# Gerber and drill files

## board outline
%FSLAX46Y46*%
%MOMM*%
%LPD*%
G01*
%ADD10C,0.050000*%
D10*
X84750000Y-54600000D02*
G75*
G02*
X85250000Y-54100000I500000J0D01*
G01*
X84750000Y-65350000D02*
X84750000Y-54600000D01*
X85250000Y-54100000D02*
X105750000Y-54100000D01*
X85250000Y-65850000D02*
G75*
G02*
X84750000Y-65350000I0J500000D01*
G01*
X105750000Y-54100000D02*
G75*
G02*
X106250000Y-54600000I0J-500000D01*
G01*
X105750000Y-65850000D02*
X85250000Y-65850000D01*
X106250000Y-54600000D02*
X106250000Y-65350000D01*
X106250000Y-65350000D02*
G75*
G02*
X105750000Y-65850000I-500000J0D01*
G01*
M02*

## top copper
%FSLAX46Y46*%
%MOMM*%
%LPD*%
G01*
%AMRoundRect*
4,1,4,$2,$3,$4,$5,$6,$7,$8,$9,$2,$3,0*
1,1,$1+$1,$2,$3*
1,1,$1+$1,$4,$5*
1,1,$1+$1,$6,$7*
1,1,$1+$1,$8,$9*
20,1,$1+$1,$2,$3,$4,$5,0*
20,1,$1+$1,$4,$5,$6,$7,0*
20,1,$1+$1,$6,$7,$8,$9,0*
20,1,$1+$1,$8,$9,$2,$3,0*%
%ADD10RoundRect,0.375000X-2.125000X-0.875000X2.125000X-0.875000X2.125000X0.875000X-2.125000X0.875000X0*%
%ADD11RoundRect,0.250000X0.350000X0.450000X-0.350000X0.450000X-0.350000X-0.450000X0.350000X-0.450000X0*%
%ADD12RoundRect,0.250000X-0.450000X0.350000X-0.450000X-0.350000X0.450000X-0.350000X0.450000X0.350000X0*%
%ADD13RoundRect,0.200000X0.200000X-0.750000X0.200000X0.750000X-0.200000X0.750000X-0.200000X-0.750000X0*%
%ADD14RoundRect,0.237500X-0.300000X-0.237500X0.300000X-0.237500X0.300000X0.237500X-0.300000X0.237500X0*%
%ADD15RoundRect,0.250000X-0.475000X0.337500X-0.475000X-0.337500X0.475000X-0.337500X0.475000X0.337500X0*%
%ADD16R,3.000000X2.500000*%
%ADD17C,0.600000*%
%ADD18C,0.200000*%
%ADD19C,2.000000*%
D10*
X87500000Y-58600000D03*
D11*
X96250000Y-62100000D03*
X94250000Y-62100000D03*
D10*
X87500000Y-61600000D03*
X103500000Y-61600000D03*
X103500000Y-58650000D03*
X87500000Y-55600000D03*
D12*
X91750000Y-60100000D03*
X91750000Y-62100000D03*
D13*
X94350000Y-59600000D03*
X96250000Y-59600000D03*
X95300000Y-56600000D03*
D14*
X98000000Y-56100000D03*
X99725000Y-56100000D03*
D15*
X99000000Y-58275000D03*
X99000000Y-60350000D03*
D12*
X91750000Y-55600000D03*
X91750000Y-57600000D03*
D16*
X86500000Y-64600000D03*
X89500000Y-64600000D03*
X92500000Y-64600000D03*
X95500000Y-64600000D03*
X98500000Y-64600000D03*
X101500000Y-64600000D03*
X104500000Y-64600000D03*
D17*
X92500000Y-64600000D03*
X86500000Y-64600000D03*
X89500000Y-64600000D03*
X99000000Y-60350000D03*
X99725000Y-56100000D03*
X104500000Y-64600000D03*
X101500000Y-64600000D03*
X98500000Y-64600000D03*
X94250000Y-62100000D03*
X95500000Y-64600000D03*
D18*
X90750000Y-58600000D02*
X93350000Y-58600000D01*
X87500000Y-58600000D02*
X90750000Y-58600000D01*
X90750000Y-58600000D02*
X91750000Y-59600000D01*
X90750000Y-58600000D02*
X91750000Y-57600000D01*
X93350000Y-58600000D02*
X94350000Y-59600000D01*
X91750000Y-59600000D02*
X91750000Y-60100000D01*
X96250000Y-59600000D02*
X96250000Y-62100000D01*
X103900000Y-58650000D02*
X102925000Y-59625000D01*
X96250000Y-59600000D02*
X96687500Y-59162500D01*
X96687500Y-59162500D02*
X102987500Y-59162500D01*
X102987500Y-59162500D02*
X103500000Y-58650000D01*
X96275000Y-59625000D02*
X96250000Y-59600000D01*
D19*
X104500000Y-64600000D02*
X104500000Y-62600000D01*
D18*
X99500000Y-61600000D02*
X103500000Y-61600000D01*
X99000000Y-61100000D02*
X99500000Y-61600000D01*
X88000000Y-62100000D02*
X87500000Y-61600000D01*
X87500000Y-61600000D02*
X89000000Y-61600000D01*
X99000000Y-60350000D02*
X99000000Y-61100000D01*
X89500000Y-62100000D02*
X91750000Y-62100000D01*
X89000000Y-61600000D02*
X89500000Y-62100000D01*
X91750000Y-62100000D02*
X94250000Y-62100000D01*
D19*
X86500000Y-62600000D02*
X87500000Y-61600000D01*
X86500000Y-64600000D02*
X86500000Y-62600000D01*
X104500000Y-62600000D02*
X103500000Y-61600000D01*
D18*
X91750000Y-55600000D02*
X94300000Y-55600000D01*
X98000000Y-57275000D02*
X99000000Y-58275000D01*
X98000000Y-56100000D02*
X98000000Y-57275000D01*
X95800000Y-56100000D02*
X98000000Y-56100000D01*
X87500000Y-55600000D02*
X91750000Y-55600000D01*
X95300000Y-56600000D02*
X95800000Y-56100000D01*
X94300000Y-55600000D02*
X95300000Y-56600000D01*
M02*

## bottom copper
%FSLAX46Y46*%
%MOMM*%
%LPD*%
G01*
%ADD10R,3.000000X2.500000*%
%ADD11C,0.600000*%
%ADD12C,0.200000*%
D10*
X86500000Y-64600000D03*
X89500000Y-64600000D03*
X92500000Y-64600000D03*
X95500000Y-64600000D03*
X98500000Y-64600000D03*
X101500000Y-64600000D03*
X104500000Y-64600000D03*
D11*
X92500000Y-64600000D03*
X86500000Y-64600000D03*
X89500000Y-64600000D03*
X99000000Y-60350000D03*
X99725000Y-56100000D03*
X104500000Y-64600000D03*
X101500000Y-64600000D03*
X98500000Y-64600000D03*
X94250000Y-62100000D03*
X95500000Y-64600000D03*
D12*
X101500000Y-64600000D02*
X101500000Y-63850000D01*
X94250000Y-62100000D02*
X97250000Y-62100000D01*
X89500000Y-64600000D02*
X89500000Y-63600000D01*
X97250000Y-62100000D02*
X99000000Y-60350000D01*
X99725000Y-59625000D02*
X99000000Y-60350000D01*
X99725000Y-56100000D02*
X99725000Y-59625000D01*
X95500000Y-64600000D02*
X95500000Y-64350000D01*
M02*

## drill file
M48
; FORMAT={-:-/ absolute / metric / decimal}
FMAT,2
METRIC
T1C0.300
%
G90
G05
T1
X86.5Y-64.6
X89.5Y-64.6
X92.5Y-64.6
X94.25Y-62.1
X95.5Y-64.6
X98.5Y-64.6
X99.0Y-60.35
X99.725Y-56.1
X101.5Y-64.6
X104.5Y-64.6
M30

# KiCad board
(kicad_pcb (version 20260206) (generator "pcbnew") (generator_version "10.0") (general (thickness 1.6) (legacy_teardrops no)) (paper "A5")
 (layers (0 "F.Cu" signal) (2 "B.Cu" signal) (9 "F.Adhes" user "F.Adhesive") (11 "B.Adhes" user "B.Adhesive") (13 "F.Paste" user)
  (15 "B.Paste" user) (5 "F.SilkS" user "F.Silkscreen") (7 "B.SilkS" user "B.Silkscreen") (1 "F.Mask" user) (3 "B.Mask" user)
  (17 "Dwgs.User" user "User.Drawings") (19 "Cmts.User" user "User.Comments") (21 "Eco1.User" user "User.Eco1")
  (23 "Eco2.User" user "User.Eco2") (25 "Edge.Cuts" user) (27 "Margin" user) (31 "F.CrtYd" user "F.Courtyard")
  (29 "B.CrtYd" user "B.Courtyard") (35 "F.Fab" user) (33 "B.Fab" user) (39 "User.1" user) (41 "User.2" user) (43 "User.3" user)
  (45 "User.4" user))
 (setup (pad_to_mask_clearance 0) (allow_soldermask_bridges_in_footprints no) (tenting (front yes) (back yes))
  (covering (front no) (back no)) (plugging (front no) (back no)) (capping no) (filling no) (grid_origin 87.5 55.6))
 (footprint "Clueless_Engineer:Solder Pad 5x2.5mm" (layer "F.Cu") (at 87.5 58.6)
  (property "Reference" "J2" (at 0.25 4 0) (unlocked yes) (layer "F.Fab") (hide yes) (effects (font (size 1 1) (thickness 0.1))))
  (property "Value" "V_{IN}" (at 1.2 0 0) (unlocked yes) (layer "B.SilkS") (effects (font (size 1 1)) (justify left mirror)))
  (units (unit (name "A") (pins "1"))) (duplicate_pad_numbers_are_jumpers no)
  (pad "1" smd roundrect (at 0 0) (size 5 2.5) (layers "F.Cu" "F.Mask" "F.Paste") (roundrect_rratio 0.15) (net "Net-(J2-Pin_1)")))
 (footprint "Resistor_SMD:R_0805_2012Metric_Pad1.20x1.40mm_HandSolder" (layer "F.Cu") (at 95.25 62.1 180)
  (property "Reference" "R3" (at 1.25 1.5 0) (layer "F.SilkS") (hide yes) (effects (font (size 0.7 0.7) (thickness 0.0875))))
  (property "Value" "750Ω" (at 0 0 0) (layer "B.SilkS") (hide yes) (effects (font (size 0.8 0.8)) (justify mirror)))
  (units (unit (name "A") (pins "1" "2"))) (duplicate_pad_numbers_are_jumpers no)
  (pad "1" smd roundrect (at -1 0 180) (size 1.2 1.4) (layers "F.Cu" "F.Mask" "F.Paste") (roundrect_rratio 0.208333) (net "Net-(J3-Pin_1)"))
  (pad "2" smd roundrect (at 1 0 180) (size 1.2 1.4) (layers "F.Cu" "F.Mask" "F.Paste") (roundrect_rratio 0.208333) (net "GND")))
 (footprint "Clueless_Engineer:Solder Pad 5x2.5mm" (layer "F.Cu") (at 87.5 61.6)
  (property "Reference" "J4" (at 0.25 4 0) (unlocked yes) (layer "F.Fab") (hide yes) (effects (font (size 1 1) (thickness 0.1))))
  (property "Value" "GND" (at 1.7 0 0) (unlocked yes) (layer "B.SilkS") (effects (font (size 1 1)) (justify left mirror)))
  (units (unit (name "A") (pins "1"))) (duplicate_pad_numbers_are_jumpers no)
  (pad "1" smd roundrect (at 0 0) (size 5 2.5) (layers "F.Cu" "F.Mask" "F.Paste") (roundrect_rratio 0.15) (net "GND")))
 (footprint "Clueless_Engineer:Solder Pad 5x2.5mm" (layer "F.Cu") (at 103.5 61.6)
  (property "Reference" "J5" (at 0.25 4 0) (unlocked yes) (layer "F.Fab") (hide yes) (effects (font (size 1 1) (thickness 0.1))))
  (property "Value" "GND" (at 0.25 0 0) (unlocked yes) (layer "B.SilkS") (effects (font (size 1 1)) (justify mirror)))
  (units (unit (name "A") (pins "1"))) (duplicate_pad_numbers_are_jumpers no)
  (pad "1" smd roundrect (at 0 0) (size 5 2.5) (layers "F.Cu" "F.Mask" "F.Paste") (roundrect_rratio 0.15) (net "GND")))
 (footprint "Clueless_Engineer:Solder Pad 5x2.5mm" (layer "F.Cu") (at 103.6 58.85)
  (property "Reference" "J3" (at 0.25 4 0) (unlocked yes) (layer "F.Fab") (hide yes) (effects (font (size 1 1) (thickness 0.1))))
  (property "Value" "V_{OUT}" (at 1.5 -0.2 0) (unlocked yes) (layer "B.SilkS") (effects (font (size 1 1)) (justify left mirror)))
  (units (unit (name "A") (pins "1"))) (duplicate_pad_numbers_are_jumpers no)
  (pad "1" smd roundrect (at -0.1 -0.2) (size 5 2.5) (layers "F.Cu" "F.Mask" "F.Paste") (roundrect_rratio 0.15) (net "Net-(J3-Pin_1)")))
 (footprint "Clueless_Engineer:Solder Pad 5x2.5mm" (layer "F.Cu") (at 87.5 55.6)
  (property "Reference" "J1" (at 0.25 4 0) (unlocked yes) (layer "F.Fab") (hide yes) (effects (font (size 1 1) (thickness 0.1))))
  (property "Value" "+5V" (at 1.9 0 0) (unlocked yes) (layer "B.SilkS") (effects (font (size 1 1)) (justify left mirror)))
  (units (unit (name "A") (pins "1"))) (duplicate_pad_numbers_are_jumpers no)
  (pad "1" smd roundrect (at 0 0) (size 5 2.5) (layers "F.Cu" "F.Mask" "F.Paste") (roundrect_rratio 0.15) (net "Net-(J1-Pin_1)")))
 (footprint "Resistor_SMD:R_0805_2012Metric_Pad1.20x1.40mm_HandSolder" (layer "F.Cu") (at 91.75 61.1 -90)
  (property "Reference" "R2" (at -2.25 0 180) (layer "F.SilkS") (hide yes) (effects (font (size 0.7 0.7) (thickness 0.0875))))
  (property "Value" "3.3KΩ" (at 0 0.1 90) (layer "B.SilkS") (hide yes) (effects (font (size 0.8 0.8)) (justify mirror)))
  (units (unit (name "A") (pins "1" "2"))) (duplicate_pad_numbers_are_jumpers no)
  (pad "1" smd roundrect (at -1 0 270) (size 1.2 1.4) (layers "F.Cu" "F.Mask" "F.Paste") (roundrect_rratio 0.208333) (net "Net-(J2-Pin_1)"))
  (pad "2" smd roundrect (at 1 0 270) (size 1.2 1.4) (layers "F.Cu" "F.Mask" "F.Paste") (roundrect_rratio 0.208333) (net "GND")))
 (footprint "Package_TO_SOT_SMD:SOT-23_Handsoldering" (layer "F.Cu") (at 95.3 58.1 90)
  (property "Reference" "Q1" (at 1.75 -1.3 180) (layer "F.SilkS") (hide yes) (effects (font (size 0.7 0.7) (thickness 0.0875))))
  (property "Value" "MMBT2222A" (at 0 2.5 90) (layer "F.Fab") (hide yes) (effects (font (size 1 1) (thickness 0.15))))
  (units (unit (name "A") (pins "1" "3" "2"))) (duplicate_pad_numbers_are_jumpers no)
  (pad "1" smd roundrect (at -1.5 -0.95 90) (size 1.9 0.8) (layers "F.Cu" "F.Mask" "F.Paste") (roundrect_rratio 0.25) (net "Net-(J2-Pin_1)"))
  (pad "2" smd roundrect (at -1.5 0.95 90) (size 1.9 0.8) (layers "F.Cu" "F.Mask" "F.Paste") (roundrect_rratio 0.25) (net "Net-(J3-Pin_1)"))
  (pad "3" smd roundrect (at 1.5 0 90) (size 1.9 0.8) (layers "F.Cu" "F.Mask" "F.Paste") (roundrect_rratio 0.25) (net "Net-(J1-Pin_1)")))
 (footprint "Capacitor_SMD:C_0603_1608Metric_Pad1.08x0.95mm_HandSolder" (layer "F.Cu") (at 98.8625 56.1)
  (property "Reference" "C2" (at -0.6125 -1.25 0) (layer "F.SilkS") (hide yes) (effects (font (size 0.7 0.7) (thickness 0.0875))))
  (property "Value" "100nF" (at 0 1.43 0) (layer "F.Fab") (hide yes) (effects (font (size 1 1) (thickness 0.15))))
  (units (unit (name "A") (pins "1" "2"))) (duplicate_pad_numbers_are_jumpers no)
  (pad "1" smd roundrect (at -0.8625 0) (size 1.075 0.95) (layers "F.Cu" "F.Mask" "F.Paste") (roundrect_rratio 0.25) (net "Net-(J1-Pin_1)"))
  (pad "2" smd roundrect (at 0.8625 0) (size 1.075 0.95) (layers "F.Cu" "F.Mask" "F.Paste") (roundrect_rratio 0.25) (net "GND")))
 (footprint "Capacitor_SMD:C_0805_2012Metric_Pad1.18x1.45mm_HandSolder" (layer "F.Cu") (at 99 59.3125 -90)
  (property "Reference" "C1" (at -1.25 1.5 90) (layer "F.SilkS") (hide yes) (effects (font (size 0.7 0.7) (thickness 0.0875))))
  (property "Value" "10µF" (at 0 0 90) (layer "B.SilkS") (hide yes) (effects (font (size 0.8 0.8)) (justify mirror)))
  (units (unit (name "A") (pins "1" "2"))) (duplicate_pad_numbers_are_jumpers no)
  (pad "1" smd roundrect (at -1.0375 0 270) (size 1.175 1.45) (layers "F.Cu" "F.Mask" "F.Paste") (roundrect_rratio 0.212766)
   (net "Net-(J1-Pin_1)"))
  (pad "2" smd roundrect (at 1.0375 0 270) (size 1.175 1.45) (layers "F.Cu" "F.Mask" "F.Paste") (roundrect_rratio 0.212766) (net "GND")))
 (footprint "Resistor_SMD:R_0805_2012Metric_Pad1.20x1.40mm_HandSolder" (layer "F.Cu") (at 91.75 56.6 -90)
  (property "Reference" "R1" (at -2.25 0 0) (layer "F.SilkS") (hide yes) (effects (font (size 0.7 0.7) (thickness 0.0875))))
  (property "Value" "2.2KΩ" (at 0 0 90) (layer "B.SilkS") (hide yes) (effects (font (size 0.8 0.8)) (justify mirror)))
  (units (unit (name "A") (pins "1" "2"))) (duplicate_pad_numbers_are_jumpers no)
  (pad "1" smd roundrect (at -1 0 270) (size 1.2 1.4) (layers "F.Cu" "F.Mask" "F.Paste") (roundrect_rratio 0.208333) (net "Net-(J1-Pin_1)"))
  (pad "2" smd roundrect (at 1 0 270) (size 1.2 1.4) (layers "F.Cu" "F.Mask" "F.Paste") (roundrect_rratio 0.208333) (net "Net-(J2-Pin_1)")))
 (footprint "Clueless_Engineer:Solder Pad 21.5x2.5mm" (layer "F.Cu") (at 89 64.6)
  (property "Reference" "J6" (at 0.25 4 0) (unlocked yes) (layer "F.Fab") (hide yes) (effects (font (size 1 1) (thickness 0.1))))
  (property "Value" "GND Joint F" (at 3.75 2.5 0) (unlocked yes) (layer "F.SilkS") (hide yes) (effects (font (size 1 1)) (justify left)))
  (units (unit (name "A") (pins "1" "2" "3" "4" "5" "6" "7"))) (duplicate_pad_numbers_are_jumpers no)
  (pad "1" smd rect (at -2.5 0) (size 3 2.5) (layers "F.Cu" "F.Mask" "F.Paste") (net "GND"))
  (pad "2" smd rect (at 0.5 0) (size 3 2.5) (layers "F.Cu" "F.Mask" "F.Paste") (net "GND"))
  (pad "3" smd rect (at 3.5 0) (size 3 2.5) (layers "F.Cu" "F.Mask" "F.Paste") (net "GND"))
  (pad "4" smd rect (at 6.5 0) (size 3 2.5) (layers "F.Cu" "F.Mask" "F.Paste") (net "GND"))
  (pad "5" smd rect (at 9.5 0) (size 3 2.5) (layers "F.Cu" "F.Mask" "F.Paste") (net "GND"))
  (pad "6" smd rect (at 12.5 0) (size 3 2.5) (layers "F.Cu" "F.Mask" "F.Paste") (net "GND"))
  (pad "7" smd rect (at 15.5 0) (size 3 2.5) (layers "F.Cu" "F.Mask" "F.Paste") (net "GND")))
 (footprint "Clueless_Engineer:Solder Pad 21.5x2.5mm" (layer "B.Cu") (at 89 64.6)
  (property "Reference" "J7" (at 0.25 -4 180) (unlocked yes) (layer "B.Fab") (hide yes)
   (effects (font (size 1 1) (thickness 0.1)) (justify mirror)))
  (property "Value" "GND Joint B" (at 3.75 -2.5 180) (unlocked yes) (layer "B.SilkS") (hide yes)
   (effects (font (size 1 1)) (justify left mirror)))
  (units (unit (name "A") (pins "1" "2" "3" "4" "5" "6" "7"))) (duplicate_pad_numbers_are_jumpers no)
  (pad "1" smd rect (at -2.5 0) (size 3 2.5) (layers "B.Cu" "B.Mask" "B.Paste") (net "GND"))
  (pad "2" smd rect (at 0.5 0) (size 3 2.5) (layers "B.Cu" "B.Mask" "B.Paste") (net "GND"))
  (pad "3" smd rect (at 3.5 0) (size 3 2.5) (layers "B.Cu" "B.Mask" "B.Paste") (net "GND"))
  (pad "4" smd rect (at 6.5 0) (size 3 2.5) (layers "B.Cu" "B.Mask" "B.Paste") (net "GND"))
  (pad "5" smd rect (at 9.5 0) (size 3 2.5) (layers "B.Cu" "B.Mask" "B.Paste") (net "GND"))
  (pad "6" smd rect (at 12.5 0) (size 3 2.5) (layers "B.Cu" "B.Mask" "B.Paste") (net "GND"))
  (pad "7" smd rect (at 15.5 0) (size 3 2.5) (layers "B.Cu" "B.Mask" "B.Paste") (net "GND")))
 (gr_arc (start 84.75 54.6) (mid 84.896447 54.246447) (end 85.25 54.1) (stroke (width 0.05) (type default)) (layer "Edge.Cuts"))
 (gr_line (start 84.75 65.35) (end 84.75 54.6) (stroke (width 0.05) (type default)) (layer "Edge.Cuts"))
 (gr_line (start 85.25 54.1) (end 105.75 54.1) (stroke (width 0.05) (type default)) (layer "Edge.Cuts"))
 (gr_arc (start 85.25 65.85) (mid 84.896447 65.703553) (end 84.75 65.35) (stroke (width 0.05) (type default)) (layer "Edge.Cuts"))
 (gr_arc (start 105.75 54.1) (mid 106.103553 54.246447) (end 106.25 54.6) (stroke (width 0.05) (type default)) (layer "Edge.Cuts"))
 (gr_line (start 105.75 65.85) (end 85.25 65.85) (stroke (width 0.05) (type default)) (layer "Edge.Cuts"))
 (gr_line (start 106.25 54.6) (end 106.25 65.35) (stroke (width 0.05) (type default)) (layer "Edge.Cuts"))
 (gr_arc (start 106.25 65.35) (mid 106.103553 65.703553) (end 105.75 65.85) (stroke (width 0.05) (type default)) (layer "Edge.Cuts"))
 (segment (start 90.75 58.6) (end 93.35 58.6) (width 0.2) (layer "F.Cu") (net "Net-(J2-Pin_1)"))
 (segment (start 87.5 58.6) (end 90.75 58.6) (width 0.2) (layer "F.Cu") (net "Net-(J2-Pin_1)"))
 (segment (start 90.75 58.6) (end 91.75 59.6) (width 0.2) (layer "F.Cu") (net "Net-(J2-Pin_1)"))
 (segment (start 90.75 58.6) (end 91.75 57.6) (width 0.2) (layer "F.Cu") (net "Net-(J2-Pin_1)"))
 (segment (start 93.35 58.6) (end 94.35 59.6) (width 0.2) (layer "F.Cu") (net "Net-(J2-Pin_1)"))
 (segment (start 91.75 59.6) (end 91.75 60.1) (width 0.2) (layer "F.Cu") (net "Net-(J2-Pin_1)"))
 (segment (start 96.25 59.6) (end 96.25 62.1) (width 0.2) (layer "F.Cu") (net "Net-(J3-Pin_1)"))
 (segment (start 103.9 58.65) (end 102.925 59.625) (width 0.2) (layer "F.Cu") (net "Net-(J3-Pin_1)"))
 (segment (start 96.25 59.6) (end 96.6875 59.1625) (width 0.2) (layer "F.Cu") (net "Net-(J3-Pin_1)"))
 (segment (start 96.6875 59.1625) (end 102.9875 59.1625) (width 0.2) (layer "F.Cu") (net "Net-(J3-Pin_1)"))
 (segment (start 102.9875 59.1625) (end 103.5 58.65) (width 0.2) (layer "F.Cu") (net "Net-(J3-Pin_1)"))
 (segment (start 96.275 59.625) (end 96.25 59.6) (width 0.2) (layer "F.Cu") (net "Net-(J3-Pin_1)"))
 (segment (start 104.5 64.6) (end 104.5 62.6) (width 2) (layer "F.Cu") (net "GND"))
 (segment (start 99.5 61.6) (end 103.5 61.6) (width 0.2) (layer "F.Cu") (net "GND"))
 (segment (start 99 61.1) (end 99.5 61.6) (width 0.2) (layer "F.Cu") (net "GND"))
 (segment (start 88 62.1) (end 87.5 61.6) (width 0.2) (layer "F.Cu") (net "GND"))
 (segment (start 87.5 61.6) (end 89 61.6) (width 0.2) (layer "F.Cu") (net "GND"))
 (segment (start 99 60.35) (end 99 61.1) (width 0.2) (layer "F.Cu") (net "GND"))
 (segment (start 89.5 62.1) (end 91.75 62.1) (width 0.2) (layer "F.Cu") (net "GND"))
 (segment (start 89 61.6) (end 89.5 62.1) (width 0.2) (layer "F.Cu") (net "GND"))
 (segment (start 91.75 62.1) (end 94.25 62.1) (width 0.2) (layer "F.Cu") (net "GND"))
 (segment (start 86.5 62.6) (end 87.5 61.6) (width 2) (layer "F.Cu") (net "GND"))
 (segment (start 86.5 64.6) (end 86.5 62.6) (width 2) (layer "F.Cu") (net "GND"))
 (segment (start 104.5 62.6) (end 103.5 61.6) (width 2) (layer "F.Cu") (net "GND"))
 (via (at 92.5 64.6) (size 0.6) (drill 0.3) (layers "F.Cu" "B.Cu") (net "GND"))
 (via (at 86.5 64.6) (size 0.6) (drill 0.3) (layers "F.Cu" "B.Cu") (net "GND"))
 (via (at 89.5 64.6) (size 0.6) (drill 0.3) (layers "F.Cu" "B.Cu") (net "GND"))
 (via (at 99 60.35) (size 0.6) (drill 0.3) (layers "F.Cu" "B.Cu") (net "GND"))
 (via (at 99.725 56.1) (size 0.6) (drill 0.3) (layers "F.Cu" "B.Cu") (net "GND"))
 (via (at 104.5 64.6) (size 0.6) (drill 0.3) (layers "F.Cu" "B.Cu") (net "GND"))
 (via (at 101.5 64.6) (size 0.6) (drill 0.3) (layers "F.Cu" "B.Cu") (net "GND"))
 (via (at 98.5 64.6) (size 0.6) (drill 0.3) (layers "F.Cu" "B.Cu") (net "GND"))
 (via (at 94.25 62.1) (size 0.6) (drill 0.3) (layers "F.Cu" "B.Cu") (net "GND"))
 (via (at 95.5 64.6) (size 0.6) (drill 0.3) (layers "F.Cu" "B.Cu") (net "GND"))
 (segment (start 101.5 64.6) (end 101.5 63.85) (width 0.2) (layer "B.Cu") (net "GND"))
 (segment (start 94.25 62.1) (end 97.25 62.1) (width 0.2) (layer "B.Cu") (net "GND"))
 (segment (start 89.5 64.6) (end 89.5 63.6) (width 0.2) (layer "B.Cu") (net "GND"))
 (segment (start 97.25 62.1) (end 99 60.35) (width 0.2) (layer "B.Cu") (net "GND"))
 (segment (start 99.725 59.625) (end 99 60.35) (width 0.2) (layer "B.Cu") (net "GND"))
 (segment (start 99.725 56.1) (end 99.725 59.625) (width 0.2) (layer "B.Cu") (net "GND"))
 (segment (start 95.5 64.6) (end 95.5 64.35) (width 0.2) (layer "B.Cu") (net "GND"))
 (segment (start 91.75 55.6) (end 94.3 55.6) (width 0.2) (layer "F.Cu") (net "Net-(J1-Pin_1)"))
 (segment (start 98 57.275) (end 99 58.275) (width 0.2) (layer "F.Cu") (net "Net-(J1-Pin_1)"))
 (segment (start 98 56.1) (end 98 57.275) (width 0.2) (layer "F.Cu") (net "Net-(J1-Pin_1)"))
 (segment (start 95.8 56.1) (end 98 56.1) (width 0.2) (layer "F.Cu") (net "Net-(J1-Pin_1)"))
 (segment (start 87.5 55.6) (end 91.75 55.6) (width 0.2) (layer "F.Cu") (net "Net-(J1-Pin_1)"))
 (segment (start 95.3 56.6) (end 95.8 56.1) (width 0.2) (layer "F.Cu") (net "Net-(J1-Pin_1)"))
 (segment (start 94.3 55.6) (end 95.3 56.6) (width 0.2) (layer "F.Cu") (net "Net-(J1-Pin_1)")))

